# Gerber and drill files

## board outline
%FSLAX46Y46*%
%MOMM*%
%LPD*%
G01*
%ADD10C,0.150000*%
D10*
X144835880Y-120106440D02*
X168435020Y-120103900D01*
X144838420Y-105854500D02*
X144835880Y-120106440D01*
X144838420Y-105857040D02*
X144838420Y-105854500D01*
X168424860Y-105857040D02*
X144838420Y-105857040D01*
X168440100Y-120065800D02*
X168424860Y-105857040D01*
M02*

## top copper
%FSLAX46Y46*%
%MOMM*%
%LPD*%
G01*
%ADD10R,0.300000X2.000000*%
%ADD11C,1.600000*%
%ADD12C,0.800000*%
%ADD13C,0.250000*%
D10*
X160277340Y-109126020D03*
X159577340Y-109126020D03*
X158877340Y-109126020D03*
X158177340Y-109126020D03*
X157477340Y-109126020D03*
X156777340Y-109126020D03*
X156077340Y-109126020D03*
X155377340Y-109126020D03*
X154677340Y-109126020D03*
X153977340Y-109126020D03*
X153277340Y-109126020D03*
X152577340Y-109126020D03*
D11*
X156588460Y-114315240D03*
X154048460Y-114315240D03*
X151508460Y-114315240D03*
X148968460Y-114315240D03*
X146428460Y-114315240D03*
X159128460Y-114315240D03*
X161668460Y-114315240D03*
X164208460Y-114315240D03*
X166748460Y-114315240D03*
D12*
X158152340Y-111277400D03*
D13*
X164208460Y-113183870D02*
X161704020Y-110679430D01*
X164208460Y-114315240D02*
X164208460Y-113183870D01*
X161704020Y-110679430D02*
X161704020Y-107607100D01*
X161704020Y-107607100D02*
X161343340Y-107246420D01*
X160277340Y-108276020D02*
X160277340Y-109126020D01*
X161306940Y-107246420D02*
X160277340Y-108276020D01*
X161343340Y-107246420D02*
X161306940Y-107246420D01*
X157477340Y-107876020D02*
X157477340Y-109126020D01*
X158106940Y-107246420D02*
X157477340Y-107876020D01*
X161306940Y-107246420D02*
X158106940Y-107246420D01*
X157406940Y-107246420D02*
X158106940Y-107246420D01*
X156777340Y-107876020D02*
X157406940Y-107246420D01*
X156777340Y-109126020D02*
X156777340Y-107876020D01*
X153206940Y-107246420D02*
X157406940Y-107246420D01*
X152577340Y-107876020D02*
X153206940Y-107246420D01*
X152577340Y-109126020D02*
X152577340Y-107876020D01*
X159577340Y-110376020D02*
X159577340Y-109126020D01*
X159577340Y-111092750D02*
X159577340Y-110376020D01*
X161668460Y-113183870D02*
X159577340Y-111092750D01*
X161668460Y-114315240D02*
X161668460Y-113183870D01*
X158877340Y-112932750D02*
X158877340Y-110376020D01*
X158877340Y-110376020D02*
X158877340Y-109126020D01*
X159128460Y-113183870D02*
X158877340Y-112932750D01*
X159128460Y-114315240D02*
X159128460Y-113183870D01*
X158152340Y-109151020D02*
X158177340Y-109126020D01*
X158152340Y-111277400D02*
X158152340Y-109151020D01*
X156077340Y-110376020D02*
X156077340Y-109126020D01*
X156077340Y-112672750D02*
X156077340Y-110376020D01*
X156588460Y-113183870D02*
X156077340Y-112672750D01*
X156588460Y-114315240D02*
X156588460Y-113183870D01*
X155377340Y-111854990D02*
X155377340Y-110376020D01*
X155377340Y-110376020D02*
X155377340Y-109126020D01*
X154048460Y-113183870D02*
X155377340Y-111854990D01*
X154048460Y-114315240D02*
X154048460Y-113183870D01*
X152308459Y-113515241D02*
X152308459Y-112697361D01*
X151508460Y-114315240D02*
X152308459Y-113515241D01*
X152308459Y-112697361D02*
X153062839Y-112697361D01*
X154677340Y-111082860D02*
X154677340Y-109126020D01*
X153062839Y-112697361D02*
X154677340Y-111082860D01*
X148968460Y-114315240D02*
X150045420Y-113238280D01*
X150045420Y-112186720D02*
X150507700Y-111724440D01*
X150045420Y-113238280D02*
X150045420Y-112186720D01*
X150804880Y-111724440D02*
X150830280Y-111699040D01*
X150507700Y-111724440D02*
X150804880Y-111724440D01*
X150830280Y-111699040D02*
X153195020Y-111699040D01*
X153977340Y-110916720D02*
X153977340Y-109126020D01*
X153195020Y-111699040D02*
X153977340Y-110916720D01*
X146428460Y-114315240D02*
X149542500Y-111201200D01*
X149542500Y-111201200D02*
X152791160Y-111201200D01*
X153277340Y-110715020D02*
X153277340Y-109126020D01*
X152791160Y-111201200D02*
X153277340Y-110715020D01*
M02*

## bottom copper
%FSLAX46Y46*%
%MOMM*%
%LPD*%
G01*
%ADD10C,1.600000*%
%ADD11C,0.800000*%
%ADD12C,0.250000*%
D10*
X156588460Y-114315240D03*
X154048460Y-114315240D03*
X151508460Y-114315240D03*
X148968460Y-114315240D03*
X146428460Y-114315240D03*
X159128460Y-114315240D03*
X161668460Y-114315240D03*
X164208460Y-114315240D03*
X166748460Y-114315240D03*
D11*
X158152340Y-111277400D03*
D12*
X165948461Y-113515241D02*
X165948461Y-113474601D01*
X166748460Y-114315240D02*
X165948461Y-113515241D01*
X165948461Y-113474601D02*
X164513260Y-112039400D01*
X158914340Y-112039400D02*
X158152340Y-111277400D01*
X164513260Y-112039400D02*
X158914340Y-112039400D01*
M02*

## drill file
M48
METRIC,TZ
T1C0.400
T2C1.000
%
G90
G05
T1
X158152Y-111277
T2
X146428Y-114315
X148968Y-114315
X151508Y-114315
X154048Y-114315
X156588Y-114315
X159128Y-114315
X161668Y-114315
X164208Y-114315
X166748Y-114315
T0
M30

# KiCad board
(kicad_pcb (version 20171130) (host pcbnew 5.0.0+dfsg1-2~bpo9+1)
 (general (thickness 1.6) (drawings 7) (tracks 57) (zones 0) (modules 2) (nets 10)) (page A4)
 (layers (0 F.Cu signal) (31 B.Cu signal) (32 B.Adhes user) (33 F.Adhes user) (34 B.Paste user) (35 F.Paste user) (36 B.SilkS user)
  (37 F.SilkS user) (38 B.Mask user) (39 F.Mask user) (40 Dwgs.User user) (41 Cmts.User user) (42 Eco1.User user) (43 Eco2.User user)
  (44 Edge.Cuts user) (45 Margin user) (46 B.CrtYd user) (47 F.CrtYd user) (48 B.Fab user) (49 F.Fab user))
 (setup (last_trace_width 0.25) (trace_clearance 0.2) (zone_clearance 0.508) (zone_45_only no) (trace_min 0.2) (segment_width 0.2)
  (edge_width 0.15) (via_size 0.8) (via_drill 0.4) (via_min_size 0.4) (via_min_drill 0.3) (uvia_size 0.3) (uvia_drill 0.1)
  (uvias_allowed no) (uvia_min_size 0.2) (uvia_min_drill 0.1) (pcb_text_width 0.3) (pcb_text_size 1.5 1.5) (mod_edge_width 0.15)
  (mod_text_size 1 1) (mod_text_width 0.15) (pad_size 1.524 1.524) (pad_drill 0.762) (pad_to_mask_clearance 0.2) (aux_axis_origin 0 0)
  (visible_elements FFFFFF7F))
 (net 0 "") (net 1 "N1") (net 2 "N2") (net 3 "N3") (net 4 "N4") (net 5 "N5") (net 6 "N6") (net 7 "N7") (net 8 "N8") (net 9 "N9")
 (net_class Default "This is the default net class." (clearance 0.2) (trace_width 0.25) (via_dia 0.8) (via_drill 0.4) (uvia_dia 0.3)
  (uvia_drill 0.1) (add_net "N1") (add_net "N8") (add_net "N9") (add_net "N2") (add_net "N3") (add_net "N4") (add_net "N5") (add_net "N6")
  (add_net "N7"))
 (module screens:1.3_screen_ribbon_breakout (layer F.Cu) (at 156.77214 108.11002 180)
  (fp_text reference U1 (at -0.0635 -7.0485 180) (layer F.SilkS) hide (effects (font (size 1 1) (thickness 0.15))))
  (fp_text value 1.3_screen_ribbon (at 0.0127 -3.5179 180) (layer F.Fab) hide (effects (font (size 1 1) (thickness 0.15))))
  (pad 1 smd rect (at -3.5052 -1.016 180) (size 0.3 2) (layers F.Cu F.Paste F.Mask) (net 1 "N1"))
  (pad 2 smd rect (at -2.8052 -1.016 180) (size 0.3 2) (layers F.Cu F.Paste F.Mask) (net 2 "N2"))
  (pad 3 smd rect (at -2.1052 -1.016 180) (size 0.3 2) (layers F.Cu F.Paste F.Mask) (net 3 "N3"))
  (pad 4 smd rect (at -1.4052 -1.016 180) (size 0.3 2) (layers F.Cu F.Paste F.Mask) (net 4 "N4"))
  (pad 5 smd rect (at -0.7052 -1.016 180) (size 0.3 2) (layers F.Cu F.Paste F.Mask) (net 1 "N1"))
  (pad 6 smd rect (at -0.0052 -1.016 180) (size 0.3 2) (layers F.Cu F.Paste F.Mask) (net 1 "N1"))
  (pad 7 smd rect (at 0.6948 -1.016 180) (size 0.3 2) (layers F.Cu F.Paste F.Mask) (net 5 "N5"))
  (pad 8 smd rect (at 1.3948 -1.016 180) (size 0.3 2) (layers F.Cu F.Paste F.Mask) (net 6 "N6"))
  (pad 9 smd rect (at 2.0948 -1.016 180) (size 0.3 2) (layers F.Cu F.Paste F.Mask) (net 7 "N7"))
  (pad 10 smd rect (at 2.7948 -1.016 180) (size 0.3 2) (layers F.Cu F.Paste F.Mask) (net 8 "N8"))
  (pad 11 smd rect (at 3.4948 -1.016 180) (size 0.3 2) (layers F.Cu F.Paste F.Mask) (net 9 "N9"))
  (pad 12 smd rect (at 4.1948 -1.016 180) (size 0.3 2) (layers F.Cu F.Paste F.Mask) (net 1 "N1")))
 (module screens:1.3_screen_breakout (layer F.Cu) (at 156.58846 114.31524 180)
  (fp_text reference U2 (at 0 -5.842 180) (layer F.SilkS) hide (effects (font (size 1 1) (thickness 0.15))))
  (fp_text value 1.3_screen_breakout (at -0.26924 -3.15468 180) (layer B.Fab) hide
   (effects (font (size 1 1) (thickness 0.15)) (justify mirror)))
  (pad 5 thru_hole circle (at 0 0 180) (size 1.6 1.6) (drill 1) (layers *.Cu *.Mask) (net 5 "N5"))
  (pad 6 thru_hole circle (at 2.54 0 180) (size 1.6 1.6) (drill 1) (layers *.Cu *.Mask) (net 6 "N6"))
  (pad 7 thru_hole circle (at 5.08 0 180) (size 1.6 1.6) (drill 1) (layers *.Cu *.Mask) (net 7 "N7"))
  (pad 8 thru_hole circle (at 7.62 0 180) (size 1.6 1.6) (drill 1) (layers *.Cu *.Mask) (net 8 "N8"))
  (pad 9 thru_hole circle (at 10.16 0 180) (size 1.6 1.6) (drill 1) (layers *.Cu *.Mask) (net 9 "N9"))
  (pad 4 thru_hole circle (at -2.54 0 180) (size 1.6 1.6) (drill 1) (layers *.Cu *.Mask) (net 3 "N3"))
  (pad 3 thru_hole circle (at -5.08 0 180) (size 1.6 1.6) (drill 1) (layers *.Cu *.Mask) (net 2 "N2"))
  (pad 2 thru_hole circle (at -7.62 0 180) (size 1.6 1.6) (drill 1) (layers *.Cu *.Mask) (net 1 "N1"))
  (pad 1 thru_hole circle (at -10.16 0 180) (size 1.6 1.6) (drill 1) (layers *.Cu *.Mask) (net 4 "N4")))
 (gr_line (start 144.83588 120.10644) (end 168.43502 120.1039) (layer Edge.Cuts) (width 0.15))
 (gr_line (start 144.83842 105.8545) (end 144.83588 120.10644) (layer Edge.Cuts) (width 0.15))
 (gr_line (start 144.83842 105.85704) (end 144.83842 105.8545) (layer Edge.Cuts) (width 0.15))
 (gr_line (start 168.42486 105.85704) (end 144.83842 105.85704) (layer Edge.Cuts) (width 0.15))
 (gr_line (start 168.4401 120.0658) (end 168.42486 105.85704) (layer Edge.Cuts) (width 0.15))
 (segment (start 164.20846 113.18387) (end 161.70402 110.67943) (width 0.25) (layer F.Cu) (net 1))
 (segment (start 164.20846 114.31524) (end 164.20846 113.18387) (width 0.25) (layer F.Cu) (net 1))
 (segment (start 161.70402 110.67943) (end 161.70402 107.6071) (width 0.25) (layer F.Cu) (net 1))
 (segment (start 161.70402 107.6071) (end 161.34334 107.24642) (width 0.25) (layer F.Cu) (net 1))
 (segment (start 160.27734 108.27602) (end 160.27734 109.12602) (width 0.25) (layer F.Cu) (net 1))
 (segment (start 161.30694 107.24642) (end 160.27734 108.27602) (width 0.25) (layer F.Cu) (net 1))
 (segment (start 161.34334 107.24642) (end 161.30694 107.24642) (width 0.25) (layer F.Cu) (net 1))
 (segment (start 157.47734 107.87602) (end 157.47734 109.12602) (width 0.25) (layer F.Cu) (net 1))
 (segment (start 158.10694 107.24642) (end 157.47734 107.87602) (width 0.25) (layer F.Cu) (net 1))
 (segment (start 161.30694 107.24642) (end 158.10694 107.24642) (width 0.25) (layer F.Cu) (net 1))
 (segment (start 157.40694 107.24642) (end 158.10694 107.24642) (width 0.25) (layer F.Cu) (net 1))
 (segment (start 156.77734 107.87602) (end 157.40694 107.24642) (width 0.25) (layer F.Cu) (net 1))
 (segment (start 156.77734 109.12602) (end 156.77734 107.87602) (width 0.25) (layer F.Cu) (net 1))
 (segment (start 153.20694 107.24642) (end 157.40694 107.24642) (width 0.25) (layer F.Cu) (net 1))
 (segment (start 152.57734 107.87602) (end 153.20694 107.24642) (width 0.25) (layer F.Cu) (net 1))
 (segment (start 152.57734 109.12602) (end 152.57734 107.87602) (width 0.25) (layer F.Cu) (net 1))
 (segment (start 159.57734 110.37602) (end 159.57734 109.12602) (width 0.25) (layer F.Cu) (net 2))
 (segment (start 159.57734 111.09275) (end 159.57734 110.37602) (width 0.25) (layer F.Cu) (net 2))
 (segment (start 161.66846 113.18387) (end 159.57734 111.09275) (width 0.25) (layer F.Cu) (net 2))
 (segment (start 161.66846 114.31524) (end 161.66846 113.18387) (width 0.25) (layer F.Cu) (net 2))
 (segment (start 158.87734 112.93275) (end 158.87734 110.37602) (width 0.25) (layer F.Cu) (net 3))
 (segment (start 158.87734 110.37602) (end 158.87734 109.12602) (width 0.25) (layer F.Cu) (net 3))
 (segment (start 159.12846 113.18387) (end 158.87734 112.93275) (width 0.25) (layer F.Cu) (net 3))
 (segment (start 159.12846 114.31524) (end 159.12846 113.18387) (width 0.25) (layer F.Cu) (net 3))
 (segment (start 165.948461 113.515241) (end 165.948461 113.474601) (width 0.25) (layer B.Cu) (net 4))
 (segment (start 166.74846 114.31524) (end 165.948461 113.515241) (width 0.25) (layer B.Cu) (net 4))
 (segment (start 165.948461 113.474601) (end 164.51326 112.0394) (width 0.25) (layer B.Cu) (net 4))
 (via (at 158.15234 111.2774) (size 0.8) (drill 0.4) (layers F.Cu B.Cu) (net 4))
 (segment (start 158.91434 112.0394) (end 158.15234 111.2774) (width 0.25) (layer B.Cu) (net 4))
 (segment (start 164.51326 112.0394) (end 158.91434 112.0394) (width 0.25) (layer B.Cu) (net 4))
 (segment (start 158.15234 109.15102) (end 158.17734 109.12602) (width 0.25) (layer F.Cu) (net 4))
 (segment (start 158.15234 111.2774) (end 158.15234 109.15102) (width 0.25) (layer F.Cu) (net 4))
 (segment (start 156.07734 110.37602) (end 156.07734 109.12602) (width 0.25) (layer F.Cu) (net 5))
 (segment (start 156.07734 112.67275) (end 156.07734 110.37602) (width 0.25) (layer F.Cu) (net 5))
 (segment (start 156.58846 113.18387) (end 156.07734 112.67275) (width 0.25) (layer F.Cu) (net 5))
 (segment (start 156.58846 114.31524) (end 156.58846 113.18387) (width 0.25) (layer F.Cu) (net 5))
 (segment (start 155.37734 111.85499) (end 155.37734 110.37602) (width 0.25) (layer F.Cu) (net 6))
 (segment (start 155.37734 110.37602) (end 155.37734 109.12602) (width 0.25) (layer F.Cu) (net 6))
 (segment (start 154.04846 113.18387) (end 155.37734 111.85499) (width 0.25) (layer F.Cu) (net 6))
 (segment (start 154.04846 114.31524) (end 154.04846 113.18387) (width 0.25) (layer F.Cu) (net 6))
 (segment (start 152.308459 113.515241) (end 152.308459 112.697361) (width 0.25) (layer F.Cu) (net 7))
 (segment (start 151.50846 114.31524) (end 152.308459 113.515241) (width 0.25) (layer F.Cu) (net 7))
 (segment (start 152.308459 112.697361) (end 153.062839 112.697361) (width 0.25) (layer F.Cu) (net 7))
 (segment (start 154.67734 111.08286) (end 154.67734 109.12602) (width 0.25) (layer F.Cu) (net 7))
 (segment (start 153.062839 112.697361) (end 154.67734 111.08286) (width 0.25) (layer F.Cu) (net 7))
 (segment (start 148.96846 114.31524) (end 150.04542 113.23828) (width 0.25) (layer F.Cu) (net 8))
 (segment (start 150.04542 112.18672) (end 150.5077 111.72444) (width 0.25) (layer F.Cu) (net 8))
 (segment (start 150.04542 113.23828) (end 150.04542 112.18672) (width 0.25) (layer F.Cu) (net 8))
 (segment (start 150.80488 111.72444) (end 150.83028 111.69904) (width 0.25) (layer F.Cu) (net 8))
 (segment (start 150.5077 111.72444) (end 150.80488 111.72444) (width 0.25) (layer F.Cu) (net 8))
 (segment (start 150.83028 111.69904) (end 153.19502 111.69904) (width 0.25) (layer F.Cu) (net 8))
 (segment (start 153.97734 110.91672) (end 153.97734 109.12602) (width 0.25) (layer F.Cu) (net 8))
 (segment (start 153.19502 111.69904) (end 153.97734 110.91672) (width 0.25) (layer F.Cu) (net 8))
 (segment (start 146.42846 114.31524) (end 149.5425 111.2012) (width 0.25) (layer F.Cu) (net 9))
 (segment (start 149.5425 111.2012) (end 152.79116 111.2012) (width 0.25) (layer F.Cu) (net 9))
 (segment (start 153.27734 110.71502) (end 153.27734 109.12602) (width 0.25) (layer F.Cu) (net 9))
 (segment (start 152.79116 111.2012) (end 153.27734 110.71502) (width 0.25) (layer F.Cu) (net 9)))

